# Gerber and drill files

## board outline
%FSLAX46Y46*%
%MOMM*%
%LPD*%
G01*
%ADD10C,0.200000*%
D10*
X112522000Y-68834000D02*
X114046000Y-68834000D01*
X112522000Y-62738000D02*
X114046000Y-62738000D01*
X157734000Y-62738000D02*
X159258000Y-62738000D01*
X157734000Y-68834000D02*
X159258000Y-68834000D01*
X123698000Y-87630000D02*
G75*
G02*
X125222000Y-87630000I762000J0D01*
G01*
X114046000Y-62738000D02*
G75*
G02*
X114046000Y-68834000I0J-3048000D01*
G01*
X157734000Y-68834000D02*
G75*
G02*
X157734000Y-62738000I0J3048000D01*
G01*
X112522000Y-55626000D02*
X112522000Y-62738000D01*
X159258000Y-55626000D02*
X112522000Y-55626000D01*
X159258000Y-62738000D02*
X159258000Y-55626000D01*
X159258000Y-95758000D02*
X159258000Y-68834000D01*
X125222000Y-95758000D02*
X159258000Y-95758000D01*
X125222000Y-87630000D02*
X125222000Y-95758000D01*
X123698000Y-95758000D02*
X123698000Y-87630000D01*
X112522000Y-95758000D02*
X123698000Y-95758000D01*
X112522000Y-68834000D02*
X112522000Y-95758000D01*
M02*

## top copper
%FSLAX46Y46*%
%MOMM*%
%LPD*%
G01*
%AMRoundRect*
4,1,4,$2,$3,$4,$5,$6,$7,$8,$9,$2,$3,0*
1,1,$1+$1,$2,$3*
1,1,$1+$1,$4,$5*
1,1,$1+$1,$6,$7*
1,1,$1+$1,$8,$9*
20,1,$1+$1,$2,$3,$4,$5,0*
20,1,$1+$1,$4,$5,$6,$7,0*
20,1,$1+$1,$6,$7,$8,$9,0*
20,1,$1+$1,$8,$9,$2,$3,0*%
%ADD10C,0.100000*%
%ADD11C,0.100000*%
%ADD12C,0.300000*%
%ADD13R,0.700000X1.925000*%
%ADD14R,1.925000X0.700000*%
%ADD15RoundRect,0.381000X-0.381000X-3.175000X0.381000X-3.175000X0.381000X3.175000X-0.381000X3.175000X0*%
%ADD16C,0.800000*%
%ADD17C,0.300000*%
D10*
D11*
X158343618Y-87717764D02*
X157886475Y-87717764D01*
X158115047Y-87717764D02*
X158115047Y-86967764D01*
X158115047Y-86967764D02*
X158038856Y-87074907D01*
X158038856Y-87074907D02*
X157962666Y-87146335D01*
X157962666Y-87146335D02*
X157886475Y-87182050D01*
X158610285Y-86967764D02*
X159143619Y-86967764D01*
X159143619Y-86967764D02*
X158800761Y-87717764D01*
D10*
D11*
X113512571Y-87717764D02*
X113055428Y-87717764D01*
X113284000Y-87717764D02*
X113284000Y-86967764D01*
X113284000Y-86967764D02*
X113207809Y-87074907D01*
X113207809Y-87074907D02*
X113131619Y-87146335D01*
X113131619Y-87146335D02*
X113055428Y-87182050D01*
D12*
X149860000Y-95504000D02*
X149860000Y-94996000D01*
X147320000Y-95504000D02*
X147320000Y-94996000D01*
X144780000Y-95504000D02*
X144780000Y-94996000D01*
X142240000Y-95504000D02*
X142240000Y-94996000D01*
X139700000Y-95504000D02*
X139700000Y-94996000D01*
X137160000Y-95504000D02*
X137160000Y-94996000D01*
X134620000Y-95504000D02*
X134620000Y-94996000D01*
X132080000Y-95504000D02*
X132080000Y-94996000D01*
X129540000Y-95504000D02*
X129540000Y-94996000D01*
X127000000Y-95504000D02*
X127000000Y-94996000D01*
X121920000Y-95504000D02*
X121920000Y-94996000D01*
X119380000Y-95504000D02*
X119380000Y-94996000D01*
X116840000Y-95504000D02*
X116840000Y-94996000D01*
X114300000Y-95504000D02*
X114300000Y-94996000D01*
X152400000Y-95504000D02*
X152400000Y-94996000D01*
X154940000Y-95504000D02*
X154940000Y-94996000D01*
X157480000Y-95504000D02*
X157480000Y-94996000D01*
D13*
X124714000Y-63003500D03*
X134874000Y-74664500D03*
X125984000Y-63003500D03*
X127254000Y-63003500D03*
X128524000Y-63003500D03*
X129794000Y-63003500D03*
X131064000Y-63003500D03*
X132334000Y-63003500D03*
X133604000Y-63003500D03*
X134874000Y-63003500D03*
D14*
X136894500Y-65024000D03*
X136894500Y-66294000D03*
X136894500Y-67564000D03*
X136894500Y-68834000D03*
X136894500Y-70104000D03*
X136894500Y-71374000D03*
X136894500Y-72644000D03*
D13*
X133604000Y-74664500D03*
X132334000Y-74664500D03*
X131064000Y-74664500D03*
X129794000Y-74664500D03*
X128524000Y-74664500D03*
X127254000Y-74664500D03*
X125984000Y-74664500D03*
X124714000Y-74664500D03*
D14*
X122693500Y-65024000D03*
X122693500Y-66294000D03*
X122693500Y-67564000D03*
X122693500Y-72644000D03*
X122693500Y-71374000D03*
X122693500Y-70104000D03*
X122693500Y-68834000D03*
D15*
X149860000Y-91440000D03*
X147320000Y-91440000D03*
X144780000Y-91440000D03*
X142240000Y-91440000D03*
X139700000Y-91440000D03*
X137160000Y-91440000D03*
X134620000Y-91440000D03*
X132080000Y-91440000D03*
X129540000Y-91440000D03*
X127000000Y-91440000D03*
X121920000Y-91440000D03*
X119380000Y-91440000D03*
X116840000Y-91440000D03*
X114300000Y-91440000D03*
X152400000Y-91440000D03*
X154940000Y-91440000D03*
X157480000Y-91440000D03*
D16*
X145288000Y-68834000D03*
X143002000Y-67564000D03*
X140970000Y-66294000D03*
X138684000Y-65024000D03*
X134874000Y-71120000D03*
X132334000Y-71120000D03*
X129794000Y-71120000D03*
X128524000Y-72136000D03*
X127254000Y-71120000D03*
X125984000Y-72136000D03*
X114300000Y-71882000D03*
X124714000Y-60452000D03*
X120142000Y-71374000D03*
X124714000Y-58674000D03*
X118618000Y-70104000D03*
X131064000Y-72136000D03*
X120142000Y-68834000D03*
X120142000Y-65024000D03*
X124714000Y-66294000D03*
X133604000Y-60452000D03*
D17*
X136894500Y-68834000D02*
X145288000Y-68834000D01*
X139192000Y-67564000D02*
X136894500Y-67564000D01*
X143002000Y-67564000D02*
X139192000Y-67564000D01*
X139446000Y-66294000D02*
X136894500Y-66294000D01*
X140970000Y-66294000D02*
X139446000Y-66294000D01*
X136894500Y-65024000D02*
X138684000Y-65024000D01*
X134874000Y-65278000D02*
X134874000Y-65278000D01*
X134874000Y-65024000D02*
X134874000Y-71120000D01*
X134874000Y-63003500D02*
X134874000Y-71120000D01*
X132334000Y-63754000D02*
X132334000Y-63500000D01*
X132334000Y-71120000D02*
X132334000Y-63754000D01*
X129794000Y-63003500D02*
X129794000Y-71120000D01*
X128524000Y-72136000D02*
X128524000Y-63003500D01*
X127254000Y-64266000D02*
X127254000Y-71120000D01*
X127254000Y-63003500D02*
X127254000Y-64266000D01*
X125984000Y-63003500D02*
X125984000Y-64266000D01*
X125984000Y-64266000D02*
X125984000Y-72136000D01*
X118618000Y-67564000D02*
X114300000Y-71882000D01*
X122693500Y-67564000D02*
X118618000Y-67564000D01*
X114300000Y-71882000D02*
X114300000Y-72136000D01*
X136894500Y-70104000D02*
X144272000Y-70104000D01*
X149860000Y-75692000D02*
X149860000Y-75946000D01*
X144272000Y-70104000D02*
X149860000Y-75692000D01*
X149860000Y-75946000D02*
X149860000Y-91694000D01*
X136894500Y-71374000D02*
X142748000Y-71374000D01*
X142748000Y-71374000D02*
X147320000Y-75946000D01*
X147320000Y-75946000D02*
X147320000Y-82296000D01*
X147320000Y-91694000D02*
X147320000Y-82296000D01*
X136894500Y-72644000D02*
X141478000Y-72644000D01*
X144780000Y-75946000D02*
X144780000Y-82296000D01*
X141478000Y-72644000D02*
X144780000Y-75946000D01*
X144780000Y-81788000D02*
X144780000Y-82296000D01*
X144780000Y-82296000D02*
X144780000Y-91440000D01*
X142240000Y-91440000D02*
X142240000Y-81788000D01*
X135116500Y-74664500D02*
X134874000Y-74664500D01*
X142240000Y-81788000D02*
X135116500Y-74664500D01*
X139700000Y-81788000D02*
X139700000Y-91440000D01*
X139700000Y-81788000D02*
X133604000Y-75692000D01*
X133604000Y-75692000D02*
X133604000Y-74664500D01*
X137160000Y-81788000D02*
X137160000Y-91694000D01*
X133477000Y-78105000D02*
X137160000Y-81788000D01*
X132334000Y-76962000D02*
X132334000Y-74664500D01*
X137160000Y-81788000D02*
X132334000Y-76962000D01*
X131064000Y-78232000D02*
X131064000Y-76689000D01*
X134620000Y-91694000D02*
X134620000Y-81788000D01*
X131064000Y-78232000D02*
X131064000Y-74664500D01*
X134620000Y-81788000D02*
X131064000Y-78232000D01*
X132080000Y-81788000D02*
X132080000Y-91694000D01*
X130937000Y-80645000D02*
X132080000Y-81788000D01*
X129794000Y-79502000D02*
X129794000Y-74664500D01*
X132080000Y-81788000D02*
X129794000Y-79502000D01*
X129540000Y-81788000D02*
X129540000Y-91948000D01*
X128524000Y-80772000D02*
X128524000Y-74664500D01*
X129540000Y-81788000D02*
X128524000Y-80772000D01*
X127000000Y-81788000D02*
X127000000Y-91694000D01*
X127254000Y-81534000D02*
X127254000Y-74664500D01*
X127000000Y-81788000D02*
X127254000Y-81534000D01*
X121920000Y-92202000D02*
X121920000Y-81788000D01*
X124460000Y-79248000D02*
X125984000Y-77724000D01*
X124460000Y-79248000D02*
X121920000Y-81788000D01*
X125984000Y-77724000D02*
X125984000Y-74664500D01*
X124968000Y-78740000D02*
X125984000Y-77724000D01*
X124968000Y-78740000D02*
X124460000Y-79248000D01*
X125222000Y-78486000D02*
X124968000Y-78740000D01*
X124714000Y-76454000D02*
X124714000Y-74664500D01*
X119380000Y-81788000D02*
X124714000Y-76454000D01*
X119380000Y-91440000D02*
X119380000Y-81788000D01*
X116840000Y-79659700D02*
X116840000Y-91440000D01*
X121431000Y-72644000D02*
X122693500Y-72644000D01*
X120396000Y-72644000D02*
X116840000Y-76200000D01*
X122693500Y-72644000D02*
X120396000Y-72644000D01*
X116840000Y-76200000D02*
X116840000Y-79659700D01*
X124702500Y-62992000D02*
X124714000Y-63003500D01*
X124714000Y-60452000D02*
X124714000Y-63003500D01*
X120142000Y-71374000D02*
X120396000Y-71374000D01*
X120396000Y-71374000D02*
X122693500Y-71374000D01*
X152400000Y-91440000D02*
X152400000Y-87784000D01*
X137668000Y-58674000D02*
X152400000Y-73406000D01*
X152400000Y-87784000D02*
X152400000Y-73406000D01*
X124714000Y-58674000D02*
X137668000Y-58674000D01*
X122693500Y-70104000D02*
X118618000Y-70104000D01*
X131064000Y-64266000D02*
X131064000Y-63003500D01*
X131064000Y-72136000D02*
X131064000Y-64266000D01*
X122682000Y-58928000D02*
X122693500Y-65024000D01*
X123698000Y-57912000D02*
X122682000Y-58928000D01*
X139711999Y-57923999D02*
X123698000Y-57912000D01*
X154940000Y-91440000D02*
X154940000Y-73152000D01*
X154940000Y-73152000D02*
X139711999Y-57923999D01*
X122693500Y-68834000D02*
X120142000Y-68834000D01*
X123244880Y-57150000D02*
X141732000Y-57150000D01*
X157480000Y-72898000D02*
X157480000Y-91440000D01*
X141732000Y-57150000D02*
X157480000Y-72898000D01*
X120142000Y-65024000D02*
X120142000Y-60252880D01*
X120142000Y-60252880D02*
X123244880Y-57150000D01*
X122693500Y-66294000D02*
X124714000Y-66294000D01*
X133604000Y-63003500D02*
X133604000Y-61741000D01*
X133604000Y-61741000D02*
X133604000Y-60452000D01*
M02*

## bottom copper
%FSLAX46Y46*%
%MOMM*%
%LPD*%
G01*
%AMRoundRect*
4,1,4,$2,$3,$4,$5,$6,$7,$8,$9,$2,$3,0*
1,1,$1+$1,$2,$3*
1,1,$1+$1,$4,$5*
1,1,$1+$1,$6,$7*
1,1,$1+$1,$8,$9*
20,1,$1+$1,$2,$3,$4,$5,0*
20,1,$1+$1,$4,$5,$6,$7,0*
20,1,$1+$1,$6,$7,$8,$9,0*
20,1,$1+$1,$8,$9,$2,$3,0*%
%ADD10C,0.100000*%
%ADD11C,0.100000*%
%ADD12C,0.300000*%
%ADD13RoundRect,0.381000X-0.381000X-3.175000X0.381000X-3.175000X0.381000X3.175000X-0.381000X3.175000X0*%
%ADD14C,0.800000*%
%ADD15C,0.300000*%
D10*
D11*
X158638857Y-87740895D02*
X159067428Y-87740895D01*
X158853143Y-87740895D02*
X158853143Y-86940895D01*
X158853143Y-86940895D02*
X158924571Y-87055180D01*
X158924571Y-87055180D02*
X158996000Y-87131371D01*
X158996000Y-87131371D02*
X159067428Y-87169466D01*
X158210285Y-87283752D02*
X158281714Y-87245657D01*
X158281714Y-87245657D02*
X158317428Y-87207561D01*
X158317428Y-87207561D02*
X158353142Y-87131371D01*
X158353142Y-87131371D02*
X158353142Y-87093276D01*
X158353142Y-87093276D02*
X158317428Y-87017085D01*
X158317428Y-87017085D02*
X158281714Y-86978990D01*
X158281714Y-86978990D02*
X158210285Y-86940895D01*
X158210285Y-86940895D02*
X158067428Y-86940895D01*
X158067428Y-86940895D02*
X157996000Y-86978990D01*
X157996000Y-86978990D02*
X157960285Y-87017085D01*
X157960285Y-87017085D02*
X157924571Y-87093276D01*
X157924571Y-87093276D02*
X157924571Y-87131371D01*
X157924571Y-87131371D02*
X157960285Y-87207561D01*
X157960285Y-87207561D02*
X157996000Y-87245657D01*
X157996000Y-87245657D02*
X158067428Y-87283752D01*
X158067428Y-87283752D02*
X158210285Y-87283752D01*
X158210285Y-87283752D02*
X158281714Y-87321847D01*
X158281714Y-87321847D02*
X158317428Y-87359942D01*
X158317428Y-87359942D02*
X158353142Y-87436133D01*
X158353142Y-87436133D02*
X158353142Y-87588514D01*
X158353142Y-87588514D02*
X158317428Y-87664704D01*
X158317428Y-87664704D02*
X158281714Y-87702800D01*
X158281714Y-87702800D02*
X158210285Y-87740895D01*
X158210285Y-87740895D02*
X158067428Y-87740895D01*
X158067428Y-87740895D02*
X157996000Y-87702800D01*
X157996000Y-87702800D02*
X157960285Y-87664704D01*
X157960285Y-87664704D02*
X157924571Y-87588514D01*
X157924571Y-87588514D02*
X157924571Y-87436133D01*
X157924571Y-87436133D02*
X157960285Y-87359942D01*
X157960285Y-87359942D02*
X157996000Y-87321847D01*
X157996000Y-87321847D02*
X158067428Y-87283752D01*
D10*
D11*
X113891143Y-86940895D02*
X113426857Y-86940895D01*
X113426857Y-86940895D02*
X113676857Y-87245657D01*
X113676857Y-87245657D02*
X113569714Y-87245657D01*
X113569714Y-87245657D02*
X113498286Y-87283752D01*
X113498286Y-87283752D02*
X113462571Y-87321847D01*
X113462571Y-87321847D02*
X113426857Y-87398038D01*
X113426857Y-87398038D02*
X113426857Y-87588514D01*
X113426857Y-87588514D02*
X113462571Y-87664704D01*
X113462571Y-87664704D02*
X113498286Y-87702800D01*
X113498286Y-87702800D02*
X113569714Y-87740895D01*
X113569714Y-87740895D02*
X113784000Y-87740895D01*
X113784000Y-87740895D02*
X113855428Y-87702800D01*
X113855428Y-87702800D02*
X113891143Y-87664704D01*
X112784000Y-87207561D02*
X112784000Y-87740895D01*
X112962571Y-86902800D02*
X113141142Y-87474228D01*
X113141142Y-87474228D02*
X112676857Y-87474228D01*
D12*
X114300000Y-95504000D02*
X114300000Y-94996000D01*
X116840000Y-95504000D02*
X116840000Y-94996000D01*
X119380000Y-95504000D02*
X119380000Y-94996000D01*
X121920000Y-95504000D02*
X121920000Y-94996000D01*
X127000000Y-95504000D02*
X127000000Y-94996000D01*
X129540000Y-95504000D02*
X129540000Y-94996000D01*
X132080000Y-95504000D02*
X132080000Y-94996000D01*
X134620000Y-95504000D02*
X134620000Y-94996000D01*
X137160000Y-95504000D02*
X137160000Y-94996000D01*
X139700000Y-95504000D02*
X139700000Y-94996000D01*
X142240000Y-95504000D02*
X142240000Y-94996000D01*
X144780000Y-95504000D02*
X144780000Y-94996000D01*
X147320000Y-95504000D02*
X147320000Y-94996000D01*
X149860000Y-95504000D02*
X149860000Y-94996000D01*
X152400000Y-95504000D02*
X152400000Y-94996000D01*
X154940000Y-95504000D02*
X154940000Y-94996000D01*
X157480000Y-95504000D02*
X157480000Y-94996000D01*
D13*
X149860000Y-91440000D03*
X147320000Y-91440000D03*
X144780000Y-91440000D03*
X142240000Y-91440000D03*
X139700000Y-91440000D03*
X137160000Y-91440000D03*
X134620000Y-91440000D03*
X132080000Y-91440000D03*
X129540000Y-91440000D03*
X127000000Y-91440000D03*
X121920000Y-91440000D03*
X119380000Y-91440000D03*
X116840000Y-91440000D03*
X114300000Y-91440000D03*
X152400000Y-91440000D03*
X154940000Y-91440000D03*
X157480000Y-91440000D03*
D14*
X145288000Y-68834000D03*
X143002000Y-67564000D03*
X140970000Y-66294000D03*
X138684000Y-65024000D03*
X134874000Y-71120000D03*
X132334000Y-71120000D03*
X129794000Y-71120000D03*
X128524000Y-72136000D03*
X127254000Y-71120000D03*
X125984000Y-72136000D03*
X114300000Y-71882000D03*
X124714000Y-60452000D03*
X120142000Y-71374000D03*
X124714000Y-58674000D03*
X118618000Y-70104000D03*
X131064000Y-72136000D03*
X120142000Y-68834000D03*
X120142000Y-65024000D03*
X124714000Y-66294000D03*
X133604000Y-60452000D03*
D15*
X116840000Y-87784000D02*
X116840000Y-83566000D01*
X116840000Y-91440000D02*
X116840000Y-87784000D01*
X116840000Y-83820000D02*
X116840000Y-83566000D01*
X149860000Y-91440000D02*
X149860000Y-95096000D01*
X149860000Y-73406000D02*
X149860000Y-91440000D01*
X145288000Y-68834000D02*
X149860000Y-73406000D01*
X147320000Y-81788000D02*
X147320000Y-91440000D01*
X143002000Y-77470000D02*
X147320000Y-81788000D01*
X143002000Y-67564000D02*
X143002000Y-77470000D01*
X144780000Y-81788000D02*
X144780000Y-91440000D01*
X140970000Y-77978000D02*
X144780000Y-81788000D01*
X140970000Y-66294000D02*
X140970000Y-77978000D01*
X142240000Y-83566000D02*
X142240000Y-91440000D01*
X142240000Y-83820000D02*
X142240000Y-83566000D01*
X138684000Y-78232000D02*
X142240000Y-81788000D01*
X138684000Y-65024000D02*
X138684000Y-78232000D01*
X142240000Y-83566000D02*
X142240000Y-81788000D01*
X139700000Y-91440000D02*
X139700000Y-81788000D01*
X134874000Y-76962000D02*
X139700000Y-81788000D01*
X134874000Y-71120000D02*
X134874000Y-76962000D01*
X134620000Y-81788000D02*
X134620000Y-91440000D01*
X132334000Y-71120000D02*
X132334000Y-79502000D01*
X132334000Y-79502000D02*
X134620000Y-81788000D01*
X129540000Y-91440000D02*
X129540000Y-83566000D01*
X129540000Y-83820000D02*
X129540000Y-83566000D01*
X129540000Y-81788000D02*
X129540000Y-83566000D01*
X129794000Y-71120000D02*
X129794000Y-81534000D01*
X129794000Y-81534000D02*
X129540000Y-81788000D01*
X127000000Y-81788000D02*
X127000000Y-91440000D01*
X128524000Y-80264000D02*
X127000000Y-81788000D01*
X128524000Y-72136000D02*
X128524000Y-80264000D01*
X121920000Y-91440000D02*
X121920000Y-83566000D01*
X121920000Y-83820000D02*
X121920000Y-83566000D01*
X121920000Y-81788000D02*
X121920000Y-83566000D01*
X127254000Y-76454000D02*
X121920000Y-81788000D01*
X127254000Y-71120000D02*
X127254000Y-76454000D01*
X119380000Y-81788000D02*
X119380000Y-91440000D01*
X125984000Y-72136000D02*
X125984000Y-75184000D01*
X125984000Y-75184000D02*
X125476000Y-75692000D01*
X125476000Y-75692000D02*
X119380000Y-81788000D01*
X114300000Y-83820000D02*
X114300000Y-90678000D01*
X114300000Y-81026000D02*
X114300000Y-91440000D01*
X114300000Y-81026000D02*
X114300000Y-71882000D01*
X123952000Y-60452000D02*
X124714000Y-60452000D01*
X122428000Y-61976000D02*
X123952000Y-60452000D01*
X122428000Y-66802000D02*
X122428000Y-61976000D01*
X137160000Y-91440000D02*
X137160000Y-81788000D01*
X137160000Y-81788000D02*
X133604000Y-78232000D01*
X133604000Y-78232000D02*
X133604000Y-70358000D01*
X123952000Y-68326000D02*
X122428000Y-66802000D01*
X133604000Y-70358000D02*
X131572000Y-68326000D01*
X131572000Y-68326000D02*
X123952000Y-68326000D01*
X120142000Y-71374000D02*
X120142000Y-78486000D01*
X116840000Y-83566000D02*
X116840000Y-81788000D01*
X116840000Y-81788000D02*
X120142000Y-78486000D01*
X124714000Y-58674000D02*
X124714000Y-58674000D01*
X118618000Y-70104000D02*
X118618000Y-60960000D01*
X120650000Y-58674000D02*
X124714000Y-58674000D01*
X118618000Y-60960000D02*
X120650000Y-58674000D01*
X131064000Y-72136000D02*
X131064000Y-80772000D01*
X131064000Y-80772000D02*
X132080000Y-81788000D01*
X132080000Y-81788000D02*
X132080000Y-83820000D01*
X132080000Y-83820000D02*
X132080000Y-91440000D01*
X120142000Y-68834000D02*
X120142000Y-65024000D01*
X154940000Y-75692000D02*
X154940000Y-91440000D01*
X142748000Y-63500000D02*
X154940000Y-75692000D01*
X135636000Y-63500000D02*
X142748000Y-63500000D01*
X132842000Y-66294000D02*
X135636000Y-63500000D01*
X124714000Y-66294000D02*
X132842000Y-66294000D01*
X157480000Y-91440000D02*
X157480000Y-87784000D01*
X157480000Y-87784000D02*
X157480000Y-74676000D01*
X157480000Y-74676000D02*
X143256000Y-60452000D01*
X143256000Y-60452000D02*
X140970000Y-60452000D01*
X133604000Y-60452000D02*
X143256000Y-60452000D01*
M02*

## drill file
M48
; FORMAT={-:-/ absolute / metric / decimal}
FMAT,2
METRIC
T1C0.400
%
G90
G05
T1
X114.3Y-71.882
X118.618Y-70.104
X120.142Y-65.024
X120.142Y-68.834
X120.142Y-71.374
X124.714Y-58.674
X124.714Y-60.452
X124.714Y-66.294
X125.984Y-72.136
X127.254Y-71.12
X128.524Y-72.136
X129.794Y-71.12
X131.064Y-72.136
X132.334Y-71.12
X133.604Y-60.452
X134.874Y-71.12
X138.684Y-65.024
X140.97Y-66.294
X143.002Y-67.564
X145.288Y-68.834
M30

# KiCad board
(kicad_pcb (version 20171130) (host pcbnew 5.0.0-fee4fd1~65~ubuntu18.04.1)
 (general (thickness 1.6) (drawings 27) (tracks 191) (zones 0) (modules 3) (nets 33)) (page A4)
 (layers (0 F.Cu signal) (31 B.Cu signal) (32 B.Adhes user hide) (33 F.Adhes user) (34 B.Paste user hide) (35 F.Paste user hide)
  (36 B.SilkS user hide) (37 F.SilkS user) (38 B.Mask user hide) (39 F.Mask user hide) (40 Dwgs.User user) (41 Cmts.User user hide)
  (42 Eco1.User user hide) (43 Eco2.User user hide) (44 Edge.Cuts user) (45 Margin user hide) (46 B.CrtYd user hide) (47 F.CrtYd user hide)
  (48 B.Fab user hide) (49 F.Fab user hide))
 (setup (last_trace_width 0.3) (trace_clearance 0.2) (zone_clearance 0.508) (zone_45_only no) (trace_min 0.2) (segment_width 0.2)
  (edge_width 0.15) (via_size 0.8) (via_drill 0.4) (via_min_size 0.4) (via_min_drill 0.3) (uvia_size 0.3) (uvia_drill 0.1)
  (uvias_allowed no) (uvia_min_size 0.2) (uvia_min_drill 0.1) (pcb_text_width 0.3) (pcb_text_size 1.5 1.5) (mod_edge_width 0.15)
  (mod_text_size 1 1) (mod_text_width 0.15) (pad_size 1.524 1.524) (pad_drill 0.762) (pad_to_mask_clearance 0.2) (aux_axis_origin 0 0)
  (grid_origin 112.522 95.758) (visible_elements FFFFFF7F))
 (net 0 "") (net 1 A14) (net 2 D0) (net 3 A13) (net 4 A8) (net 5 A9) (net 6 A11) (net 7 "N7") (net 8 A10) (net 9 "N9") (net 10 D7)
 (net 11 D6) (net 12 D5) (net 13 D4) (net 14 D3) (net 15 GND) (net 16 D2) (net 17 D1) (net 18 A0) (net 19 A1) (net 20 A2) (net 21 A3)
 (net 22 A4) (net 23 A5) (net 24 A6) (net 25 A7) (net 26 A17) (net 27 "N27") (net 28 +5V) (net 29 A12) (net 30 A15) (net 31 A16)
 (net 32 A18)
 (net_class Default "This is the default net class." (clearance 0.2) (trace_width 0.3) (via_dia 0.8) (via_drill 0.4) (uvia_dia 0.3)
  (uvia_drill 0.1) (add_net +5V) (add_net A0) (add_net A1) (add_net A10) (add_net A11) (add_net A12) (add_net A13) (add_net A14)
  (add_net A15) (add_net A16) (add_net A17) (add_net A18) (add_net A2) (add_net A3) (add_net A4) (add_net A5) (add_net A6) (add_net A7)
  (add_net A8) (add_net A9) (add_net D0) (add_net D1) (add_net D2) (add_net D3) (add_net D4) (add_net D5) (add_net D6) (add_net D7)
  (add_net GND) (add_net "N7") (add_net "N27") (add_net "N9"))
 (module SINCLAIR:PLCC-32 (layer F.Cu) (at 129.794 68.834 90)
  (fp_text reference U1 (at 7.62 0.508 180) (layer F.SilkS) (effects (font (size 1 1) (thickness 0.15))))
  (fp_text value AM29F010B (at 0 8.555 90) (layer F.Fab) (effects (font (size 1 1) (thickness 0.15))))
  (pad 29 smd rect (at 5.8305 -5.08 90) (size 1.925 0.7) (layers F.Cu F.Paste F.Mask) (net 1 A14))
  (pad 13 smd rect (at -5.8305 5.08 90) (size 1.925 0.7) (layers F.Cu F.Paste F.Mask) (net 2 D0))
  (pad 28 smd rect (at 5.8305 -3.81 90) (size 1.925 0.7) (layers F.Cu F.Paste F.Mask) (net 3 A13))
  (pad 27 smd rect (at 5.8305 -2.54 90) (size 1.925 0.7) (layers F.Cu F.Paste F.Mask) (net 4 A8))
  (pad 26 smd rect (at 5.8305 -1.27 90) (size 1.925 0.7) (layers F.Cu F.Paste F.Mask) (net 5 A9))
  (pad 25 smd rect (at 5.8305 0 90) (size 1.925 0.7) (layers F.Cu F.Paste F.Mask) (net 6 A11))
  (pad 24 smd rect (at 5.8305 1.27 90) (size 1.925 0.7) (layers F.Cu F.Paste F.Mask) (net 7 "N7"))
  (pad 23 smd rect (at 5.8305 2.54 90) (size 1.925 0.7) (layers F.Cu F.Paste F.Mask) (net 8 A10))
  (pad 22 smd rect (at 5.8305 3.81 90) (size 1.925 0.7) (layers F.Cu F.Paste F.Mask) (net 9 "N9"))
  (pad 21 smd rect (at 5.8305 5.08 90) (size 1.925 0.7) (layers F.Cu F.Paste F.Mask) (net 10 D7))
  (pad 20 smd rect (at 3.81 7.1005 90) (size 0.7 1.925) (layers F.Cu F.Paste F.Mask) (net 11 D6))
  (pad 19 smd rect (at 2.54 7.1005 90) (size 0.7 1.925) (layers F.Cu F.Paste F.Mask) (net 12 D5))
  (pad 18 smd rect (at 1.27 7.1005 90) (size 0.7 1.925) (layers F.Cu F.Paste F.Mask) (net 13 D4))
  (pad 17 smd rect (at 0 7.1005 90) (size 0.7 1.925) (layers F.Cu F.Paste F.Mask) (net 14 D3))
  (pad 16 smd rect (at -1.27 7.1005 90) (size 0.7 1.925) (layers F.Cu F.Paste F.Mask) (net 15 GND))
  (pad 15 smd rect (at -2.54 7.1005 90) (size 0.7 1.925) (layers F.Cu F.Paste F.Mask) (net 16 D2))
  (pad 14 smd rect (at -3.81 7.1005 90) (size 0.7 1.925) (layers F.Cu F.Paste F.Mask) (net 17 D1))
  (pad 12 smd rect (at -5.8305 3.81 90) (size 1.925 0.7) (layers F.Cu F.Paste F.Mask) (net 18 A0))
  (pad 11 smd rect (at -5.8305 2.54 90) (size 1.925 0.7) (layers F.Cu F.Paste F.Mask) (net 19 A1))
  (pad 10 smd rect (at -5.8305 1.27 90) (size 1.925 0.7) (layers F.Cu F.Paste F.Mask) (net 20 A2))
  (pad 9 smd rect (at -5.8305 0 90) (size 1.925 0.7) (layers F.Cu F.Paste F.Mask) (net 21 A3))
  (pad 8 smd rect (at -5.8305 -1.27 90) (size 1.925 0.7) (layers F.Cu F.Paste F.Mask) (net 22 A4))
  (pad 7 smd rect (at -5.8305 -2.54 90) (size 1.925 0.7) (layers F.Cu F.Paste F.Mask) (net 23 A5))
  (pad 6 smd rect (at -5.8305 -3.81 90) (size 1.925 0.7) (layers F.Cu F.Paste F.Mask) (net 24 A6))
  (pad 5 smd rect (at -5.8305 -5.08 90) (size 1.925 0.7) (layers F.Cu F.Paste F.Mask) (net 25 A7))
  (pad 30 smd rect (at 3.81 -7.1005 90) (size 0.7 1.925) (layers F.Cu F.Paste F.Mask) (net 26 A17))
  (pad 31 smd rect (at 2.54 -7.1005 90) (size 0.7 1.925) (layers F.Cu F.Paste F.Mask) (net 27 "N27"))
  (pad 32 smd rect (at 1.27 -7.1005 90) (size 0.7 1.925) (layers F.Cu F.Paste F.Mask) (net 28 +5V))
  (pad 4 smd rect (at -3.81 -7.1005 90) (size 0.7 1.925) (layers F.Cu F.Paste F.Mask) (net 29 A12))
  (pad 3 smd rect (at -2.54 -7.1005 90) (size 0.7 1.925) (layers F.Cu F.Paste F.Mask) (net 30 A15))
  (pad 2 smd rect (at -1.27 -7.1005 90) (size 0.7 1.925) (layers F.Cu F.Paste F.Mask) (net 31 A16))
  (pad 1 smd rect (at 0 -7.1005 90) (size 0.7 1.925) (layers F.Cu F.Paste F.Mask) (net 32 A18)))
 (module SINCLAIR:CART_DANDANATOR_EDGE (layer F.Cu) (at 124.46 91.44)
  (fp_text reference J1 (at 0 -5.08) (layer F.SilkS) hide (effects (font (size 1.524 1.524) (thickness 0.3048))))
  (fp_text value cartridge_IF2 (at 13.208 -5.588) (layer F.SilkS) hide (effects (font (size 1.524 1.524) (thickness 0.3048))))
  (fp_line (start -10.16 4.064) (end -10.16 3.556) (layer B.Cu) (width 0.3))
  (fp_line (start -7.62 4.064) (end -7.62 3.556) (layer B.Cu) (width 0.3))
  (fp_line (start -5.08 4.064) (end -5.08 3.556) (layer B.Cu) (width 0.3))
  (fp_line (start -2.54 4.064) (end -2.54 3.556) (layer B.Cu) (width 0.3))
  (fp_line (start 2.54 4.064) (end 2.54 3.556) (layer B.Cu) (width 0.3))
  (fp_line (start 5.08 4.064) (end 5.08 3.556) (layer B.Cu) (width 0.3))
  (fp_line (start 7.62 4.064) (end 7.62 3.556) (layer B.Cu) (width 0.3))
  (fp_line (start 10.16 4.064) (end 10.16 3.556) (layer B.Cu) (width 0.3))
  (fp_line (start 12.7 4.064) (end 12.7 3.556) (layer B.Cu) (width 0.3))
  (fp_line (start 15.24 4.064) (end 15.24 3.556) (layer B.Cu) (width 0.3))
  (fp_line (start 17.78 4.064) (end 17.78 3.556) (layer B.Cu) (width 0.3))
  (fp_line (start 20.32 4.064) (end 20.32 3.556) (layer B.Cu) (width 0.3))
  (fp_line (start 22.86 4.064) (end 22.86 3.556) (layer B.Cu) (width 0.3))
  (fp_line (start 25.4 4.064) (end 25.4 3.556) (layer B.Cu) (width 0.3))
  (fp_line (start 25.4 4.064) (end 25.4 3.556) (layer F.Cu) (width 0.3))
  (fp_line (start 22.86 4.064) (end 22.86 3.556) (layer F.Cu) (width 0.3))
  (fp_line (start 20.32 4.064) (end 20.32 3.556) (layer F.Cu) (width 0.3))
  (fp_line (start 17.78 4.064) (end 17.78 3.556) (layer F.Cu) (width 0.3))
  (fp_line (start 15.24 4.064) (end 15.24 3.556) (layer F.Cu) (width 0.3))
  (fp_line (start 12.7 4.064) (end 12.7 3.556) (layer F.Cu) (width 0.3))
  (fp_line (start 10.16 4.064) (end 10.16 3.556) (layer F.Cu) (width 0.3))
  (fp_line (start 7.62 4.064) (end 7.62 3.556) (layer F.Cu) (width 0.3))
  (fp_line (start 5.08 4.064) (end 5.08 3.556) (layer F.Cu) (width 0.3))
  (fp_line (start 2.54 4.064) (end 2.54 3.556) (layer F.Cu) (width 0.3))
  (fp_line (start -2.54 4.064) (end -2.54 3.556) (layer F.Cu) (width 0.3))
  (fp_line (start -5.08 4.064) (end -5.08 3.556) (layer F.Cu) (width 0.3))
  (fp_line (start -7.62 4.064) (end -7.62 3.556) (layer F.Cu) (width 0.3))
  (fp_line (start -10.16 4.064) (end -10.16 3.556) (layer F.Cu) (width 0.3))
  (fp_line (start 27.94 4.064) (end 27.94 3.556) (layer F.Cu) (width 0.3))
  (fp_line (start 30.48 4.064) (end 30.48 3.556) (layer F.Cu) (width 0.3))
  (fp_line (start 33.02 4.064) (end 33.02 3.556) (layer F.Cu) (width 0.3))
  (fp_line (start 27.94 4.064) (end 27.94 3.556) (layer B.Cu) (width 0.3))
  (fp_line (start 30.48 4.064) (end 30.48 3.556) (layer B.Cu) (width 0.3))
  (fp_line (start 33.02 4.064) (end 33.02 3.556) (layer B.Cu) (width 0.3))
  (pad 28 connect roundrect (at 25.4 0) (size 1.524 7.112) (layers B.Cu) (roundrect_rratio 0.25) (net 14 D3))
  (pad 26 connect roundrect (at 22.86 0) (size 1.524 7.112) (layers B.Cu) (roundrect_rratio 0.25) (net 13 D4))
  (pad 24 connect roundrect (at 20.32 0) (size 1.524 7.112) (layers B.Cu) (roundrect_rratio 0.25) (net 12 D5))
  (pad 22 connect roundrect (at 17.78 0) (size 1.524 7.112) (layers B.Cu) (roundrect_rratio 0.25) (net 11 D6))
  (pad 20 connect roundrect (at 15.24 0) (size 1.524 7.112) (layers B.Cu) (roundrect_rratio 0.25) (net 10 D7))
  (pad 18 connect roundrect (at 12.7 0) (size 1.524 7.112) (layers B.Cu) (roundrect_rratio 0.25) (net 1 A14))
  (pad 16 connect roundrect (at 10.16 0) (size 1.524 7.112) (layers B.Cu) (roundrect_rratio 0.25) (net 8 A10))
  (pad 14 connect roundrect (at 7.62 0) (size 1.524 7.112) (layers B.Cu) (roundrect_rratio 0.25) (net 7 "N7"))
  (pad 12 connect roundrect (at 5.08 0) (size 1.524 7.112) (layers B.Cu) (roundrect_rratio 0.25) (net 6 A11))
  (pad 10 connect roundrect (at 2.54 0) (size 1.524 7.112) (layers B.Cu) (roundrect_rratio 0.25) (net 5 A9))
  (pad 8 connect roundrect (at -2.54 0) (size 1.524 7.112) (layers B.Cu) (roundrect_rratio 0.25) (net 4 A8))
  (pad 6 connect roundrect (at -5.08 0) (size 1.524 7.112) (layers B.Cu) (roundrect_rratio 0.25) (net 3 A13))
  (pad 4 connect roundrect (at -7.62 0) (size 1.524 7.112) (layers B.Cu) (roundrect_rratio 0.25) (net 30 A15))
  (pad 2 connect roundrect (at -10.16 0) (size 1.524 7.112) (layers B.Cu) (roundrect_rratio 0.25) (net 28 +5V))
  (pad 27 connect roundrect (at 25.4 0) (size 1.524 7.112) (layers F.Cu) (roundrect_rratio 0.25) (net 15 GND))
  (pad 25 connect roundrect (at 22.86 0) (size 1.524 7.112) (layers F.Cu) (roundrect_rratio 0.25) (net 16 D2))
  (pad 23 connect roundrect (at 20.32 0) (size 1.524 7.112) (layers F.Cu) (roundrect_rratio 0.25) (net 17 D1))
  (pad 21 connect roundrect (at 17.78 0) (size 1.524 7.112) (layers F.Cu) (roundrect_rratio 0.25) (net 2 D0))
  (pad 19 connect roundrect (at 15.24 0) (size 1.524 7.112) (layers F.Cu) (roundrect_rratio 0.25) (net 18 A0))
  (pad 17 connect roundrect (at 12.7 0) (size 1.524 7.112) (layers F.Cu) (roundrect_rratio 0.25) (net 19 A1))
  (pad 15 connect roundrect (at 10.16 0) (size 1.524 7.112) (layers F.Cu) (roundrect_rratio 0.25) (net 20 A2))
  (pad 13 connect roundrect (at 7.62 0) (size 1.524 7.112) (layers F.Cu) (roundrect_rratio 0.25) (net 21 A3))
  (pad 11 connect roundrect (at 5.08 0) (size 1.524 7.112) (layers F.Cu) (roundrect_rratio 0.25) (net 22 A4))
  (pad 9 connect roundrect (at 2.54 0) (size 1.524 7.112) (layers F.Cu) (roundrect_rratio 0.25) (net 23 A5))
  (pad 7 connect roundrect (at -2.54 0) (size 1.524 7.112) (layers F.Cu) (roundrect_rratio 0.25) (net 24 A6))
  (pad 5 connect roundrect (at -5.08 0) (size 1.524 7.112) (layers F.Cu) (roundrect_rratio 0.25) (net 25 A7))
  (pad 3 connect roundrect (at -7.62 0) (size 1.524 7.112) (layers F.Cu) (roundrect_rratio 0.25) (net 29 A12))
  (pad 1 connect roundrect (at -10.16 0) (size 1.524 7.112) (layers F.Cu) (roundrect_rratio 0.25))
  (pad 29 connect roundrect (at 27.94 0) (size 1.524 7.112) (layers F.Cu) (roundrect_rratio 0.25) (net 31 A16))
  (pad 31 connect roundrect (at 30.48 0) (size 1.524 7.112) (layers F.Cu) (roundrect_rratio 0.25) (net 26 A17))
  (pad 33 connect roundrect (at 33.02 0) (size 1.524 7.112) (layers F.Cu) (roundrect_rratio 0.25) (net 32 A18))
  (pad 30 connect roundrect (at 27.94 0) (size 1.524 7.112) (layers B.Cu) (roundrect_rratio 0.25))
  (pad 32 connect roundrect (at 30.48 0) (size 1.524 7.112) (layers B.Cu) (roundrect_rratio 0.25) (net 27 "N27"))
  (pad 34 connect roundrect (at 33.02 0) (size 1.524 7.112) (layers B.Cu) (roundrect_rratio 0.25) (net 9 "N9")))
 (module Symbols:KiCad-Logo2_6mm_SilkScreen (layer F.Cu) (at 148.082 73.914)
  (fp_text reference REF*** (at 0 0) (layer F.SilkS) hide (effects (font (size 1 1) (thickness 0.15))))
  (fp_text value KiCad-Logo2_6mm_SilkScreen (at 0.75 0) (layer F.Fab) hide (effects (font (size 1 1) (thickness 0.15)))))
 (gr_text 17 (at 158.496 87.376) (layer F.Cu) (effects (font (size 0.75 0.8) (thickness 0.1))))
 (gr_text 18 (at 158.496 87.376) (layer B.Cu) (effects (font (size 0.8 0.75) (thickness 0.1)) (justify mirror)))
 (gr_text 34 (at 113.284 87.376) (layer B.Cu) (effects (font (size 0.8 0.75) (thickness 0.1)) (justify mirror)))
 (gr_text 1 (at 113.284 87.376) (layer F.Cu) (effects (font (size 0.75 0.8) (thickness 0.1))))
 (gr_line (start 112.522 68.834) (end 114.046 68.834) (layer Edge.Cuts) (width 0.2))
 (gr_line (start 112.522 62.738) (end 114.046 62.738) (layer Edge.Cuts) (width 0.2))
 (gr_line (start 157.734 62.738) (end 159.258 62.738) (layer Edge.Cuts) (width 0.2))
 (gr_line (start 157.734 68.834) (end 159.258 68.834) (layer Edge.Cuts) (width 0.2))
 (gr_arc (start 124.46 87.63) (end 125.222 87.63) (angle -180) (layer Edge.Cuts) (width 0.2))
 (gr_arc (start 114.046 65.786) (end 114.046 68.834) (angle -180) (layer Edge.Cuts) (width 0.2))
 (gr_arc (start 157.734 65.786) (end 157.734 62.738) (angle -180) (layer Edge.Cuts) (width 0.2))
 (gr_line (start 112.522 55.626) (end 112.522 62.738) (layer Edge.Cuts) (width 0.2))
 (gr_line (start 159.258 55.626) (end 112.522 55.626) (layer Edge.Cuts) (width 0.2))
 (gr_line (start 159.258 62.738) (end 159.258 55.626) (layer Edge.Cuts) (width 0.2))
 (gr_line (start 159.258 95.758) (end 159.258 68.834) (layer Edge.Cuts) (width 0.2))
 (gr_line (start 125.222 95.758) (end 159.258 95.758) (layer Edge.Cuts) (width 0.2))
 (gr_line (start 125.222 87.63) (end 125.222 95.758) (layer Edge.Cuts) (width 0.2))
 (gr_line (start 123.698 95.758) (end 123.698 87.63) (layer Edge.Cuts) (width 0.2))
 (gr_line (start 112.522 95.758) (end 123.698 95.758) (layer Edge.Cuts) (width 0.2))
 (gr_line (start 112.522 68.834) (end 112.522 95.758) (layer Edge.Cuts) (width 0.2))
 (segment (start 116.84 87.784) (end 116.84 83.566) (width 0.3) (layer B.Cu) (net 30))
 (segment (start 116.84 91.44) (end 116.84 87.784) (width 0.3) (layer B.Cu) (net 30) (status 10))
 (segment (start 116.84 83.82) (end 116.84 83.566) (width 0.3) (layer B.Cu) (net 30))
 (segment (start 149.86 91.44) (end 149.86 95.096) (width 0.3) (layer B.Cu) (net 14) (status 10))
 (segment (start 136.8945 68.834) (end 145.288 68.834) (width 0.3) (layer F.Cu) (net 14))
 (via (at 145.288 68.834) (size 0.8) (drill 0.4) (layers F.Cu B.Cu) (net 14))
 (segment (start 149.86 73.406) (end 149.86 91.44) (width 0.3) (layer B.Cu) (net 14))
 (segment (start 145.288 68.834) (end 149.86 73.406) (width 0.3) (layer B.Cu) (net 14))
 (segment (start 147.32 81.788) (end 147.32 91.44) (width 0.3) (layer B.Cu) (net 13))
 (segment (start 139.192 67.564) (end 136.8945 67.564) (width 0.3) (layer F.Cu) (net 13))
 (via (at 143.002 67.564) (size 0.8) (drill 0.4) (layers F.Cu B.Cu) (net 13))
 (segment (start 143.002 67.564) (end 139.192 67.564) (width 0.3) (layer F.Cu) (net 13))
 (segment (start 143.002 77.47) (end 147.32 81.788) (width 0.3) (layer B.Cu) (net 13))
 (segment (start 143.002 67.564) (end 143.002 77.47) (width 0.3) (layer B.Cu) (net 13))
 (via (at 140.97 66.294) (size 0.8) (drill 0.4) (layers F.Cu B.Cu) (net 12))
 (segment (start 139.446 66.294) (end 136.8945 66.294) (width 0.3) (layer F.Cu) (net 12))
 (segment (start 140.97 66.294) (end 139.446 66.294) (width 0.3) (layer F.Cu) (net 12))
 (segment (start 144.78 81.788) (end 144.78 91.44) (width 0.3) (layer B.Cu) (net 12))
 (segment (start 140.97 77.978) (end 144.78 81.788) (width 0.3) (layer B.Cu) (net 12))
 (segment (start 140.97 66.294) (end 140.97 77.978) (width 0.3) (layer B.Cu) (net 12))
 (segment (start 142.24 83.566) (end 142.24 91.44) (width 0.3) (layer B.Cu) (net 11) (status 20))
 (segment (start 142.24 83.82) (end 142.24 83.566) (width 0.3) (layer B.Cu) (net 11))
 (via (at 138.684 65.024) (size 0.8) (drill 0.4) (layers F.Cu B.Cu) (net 11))
 (segment (start 136.8945 65.024) (end 138.684 65.024) (width 0.3) (layer F.Cu) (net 11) (status 10))
 (segment (start 138.684 78.232) (end 142.24 81.788) (width 0.3) (layer B.Cu) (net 11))
 (segment (start 138.684 65.024) (end 138.684 78.232) (width 0.3) (layer B.Cu) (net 11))
 (segment (start 142.24 83.566) (end 142.24 81.788) (width 0.3) (layer B.Cu) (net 11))
 (segment (start 134.874 65.278) (end 134.874 65.278) (width 0.3) (layer F.Cu) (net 10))
 (segment (start 139.7 91.44) (end 139.7 81.788) (width 0.3) (layer B.Cu) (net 10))
 (segment (start 134.874 65.024) (end 134.874 71.12) (width 0.3) (layer F.Cu) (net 10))
 (via (at 134.874 71.12) (size 0.8) (drill 0.4) (layers F.Cu B.Cu) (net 10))
 (segment (start 134.874 63.0035) (end 134.874 71.12) (width 0.3) (layer F.Cu) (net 10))
 (segment (start 134.874 76.962) (end 139.7 81.788) (width 0.3) (layer B.Cu) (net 10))
 (segment (start 134.874 71.12) (end 134.874 76.962) (width 0.3) (layer B.Cu) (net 10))
 (segment (start 134.62 81.788) (end 134.62 91.44) (width 0.3) (layer B.Cu) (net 8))
 (segment (start 132.334 71.12) (end 132.334 79.502) (width 0.3) (layer B.Cu) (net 8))
 (segment (start 132.334 63.754) (end 132.334 63.5) (width 0.3) (layer F.Cu) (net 8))
 (segment (start 132.334 79.502) (end 134.62 81.788) (width 0.3) (layer B.Cu) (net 8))
 (via (at 132.334 71.12) (size 0.8) (drill 0.4) (layers F.Cu B.Cu) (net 8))
 (segment (start 132.334 71.12) (end 132.334 63.754) (width 0.3) (layer F.Cu) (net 8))
 (segment (start 129.54 91.44) (end 129.54 83.566) (width 0.3) (layer B.Cu) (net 6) (status 10))
 (segment (start 129.54 83.82) (end 129.54 83.566) (width 0.3) (layer B.Cu) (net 6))
 (segment (start 129.54 81.788) (end 129.54 83.566) (width 0.3) (layer B.Cu) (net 6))
 (segment (start 129.794 71.12) (end 129.794 81.534) (width 0.3) (layer B.Cu) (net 6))
 (via (at 129.794 71.12) (size 0.8) (drill 0.4) (layers F.Cu B.Cu) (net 6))
 (segment (start 129.794 81.534) (end 129.54 81.788) (width 0.3) (layer B.Cu) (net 6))
 (segment (start 129.794 63.0035) (end 129.794 71.12) (width 0.3) (layer F.Cu) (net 6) (status 10))
 (segment (start 127 81.788) (end 127 91.44) (width 0.3) (layer B.Cu) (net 5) (status 20))
 (segment (start 128.524 80.264) (end 127 81.788) (width 0.3) (layer B.Cu) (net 5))
 (via (at 128.524 72.136) (size 0.8) (drill 0.4) (layers F.Cu B.Cu) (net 5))
 (segment (start 128.524 72.136) (end 128.524 80.264) (width 0.3) (layer B.Cu) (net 5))
 (segment (start 128.524 72.136) (end 128.524 63.0035) (width 0.3) (layer F.Cu) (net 5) (status 20))
 (segment (start 121.92 91.44) (end 121.92 83.566) (width 0.3) (layer B.Cu) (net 4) (status 10))
 (segment (start 121.92 83.82) (end 121.92 83.566) (width 0.3) (layer B.Cu) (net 4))
 (segment (start 121.92 81.788) (end 121.92 83.566) (width 0.3) (layer B.Cu) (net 4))
 (segment (start 127.254 76.454) (end 121.92 81.788) (width 0.3) (layer B.Cu) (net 4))
 (segment (start 127.254 71.12) (end 127.254 76.454) (width 0.3) (layer B.Cu) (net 4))
 (via (at 127.254 71.12) (size 0.8) (drill 0.4) (layers F.Cu B.Cu) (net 4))
 (segment (start 127.254 64.266) (end 127.254 71.12) (width 0.3) (layer F.Cu) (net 4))
 (segment (start 127.254 63.0035) (end 127.254 64.266) (width 0.3) (layer F.Cu) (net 4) (status 10))
 (segment (start 119.38 81.788) (end 119.38 91.44) (width 0.3) (layer B.Cu) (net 3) (status 20))
 (via (at 125.984 72.136) (size 0.8) (drill 0.4) (layers F.Cu B.Cu) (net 3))
 (segment (start 125.984 63.0035) (end 125.984 64.266) (width 0.3) (layer F.Cu) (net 3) (status 10))
 (segment (start 125.984 64.266) (end 125.984 72.136) (width 0.3) (layer F.Cu) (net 3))
 (segment (start 125.984 72.136) (end 125.984 75.184) (width 0.3) (layer B.Cu) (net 3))
 (segment (start 125.984 75.184) (end 125.476 75.692) (width 0.3) (layer B.Cu) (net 3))
 (segment (start 125.476 75.692) (end 119.38 81.788) (width 0.3) (layer B.Cu) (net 3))
 (segment (start 114.3 83.82) (end 114.3 90.678) (width 0.3) (layer B.Cu) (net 28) (status 20))
 (segment (start 118.618 67.564) (end 114.3 71.882) (width 0.3) (layer F.Cu) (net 28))
 (segment (start 122.6935 67.564) (end 118.618 67.564) (width 0.3) (layer F.Cu) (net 28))
 (segment (start 114.3 81.026) (end 114.3 91.44) (width 0.3) (layer B.Cu) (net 28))
 (segment (start 114.3 71.882) (end 114.3 72.136) (width 0.3) (layer F.Cu) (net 28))
 (via (at 114.3 71.882) (size 0.8) (drill 0.4) (layers F.Cu B.Cu) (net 28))
 (segment (start 114.3 81.026) (end 114.3 71.882) (width 0.3) (layer B.Cu) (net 28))
 (segment (start 136.8945 70.104) (end 144.272 70.104) (width 0.3) (layer F.Cu) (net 15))
 (segment (start 149.86 75.692) (end 149.86 75.946) (width 0.3) (layer F.Cu) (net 15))
 (segment (start 144.272 70.104) (end 149.86 75.692) (width 0.3) (layer F.Cu) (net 15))
 (segment (start 149.86 75.946) (end 149.86 91.694) (width 0.3) (layer F.Cu) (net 15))
 (segment (start 136.8945 71.374) (end 142.748 71.374) (width 0.3) (layer F.Cu) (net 16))
 (segment (start 142.748 71.374) (end 147.32 75.946) (width 0.3) (layer F.Cu) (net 16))
 (segment (start 147.32 75.946) (end 147.32 82.296) (width 0.3) (layer F.Cu) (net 16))
 (segment (start 147.32 91.694) (end 147.32 82.296) (width 0.3) (layer F.Cu) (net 16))
 (segment (start 136.8945 72.644) (end 141.478 72.644) (width 0.3) (layer F.Cu) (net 17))
 (segment (start 144.78 75.946) (end 144.78 82.296) (width 0.3) (layer F.Cu) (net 17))
 (segment (start 141.478 72.644) (end 144.78 75.946) (width 0.3) (layer F.Cu) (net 17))
 (segment (start 144.78 81.788) (end 144.78 82.296) (width 0.3) (layer F.Cu) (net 17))
 (segment (start 144.78 82.296) (end 144.78 91.44) (width 0.3) (layer F.Cu) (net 17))
 (segment (start 142.24 91.44) (end 142.24 81.788) (width 0.3) (layer F.Cu) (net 2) (status 10))
 (segment (start 135.1165 74.6645) (end 134.874 74.6645) (width 0.3) (layer F.Cu) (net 2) (status 30))
 (segment (start 142.24 81.788) (end 135.1165 74.6645) (width 0.3) (layer F.Cu) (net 2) (status 20))
 (segment (start 139.7 81.788) (end 139.7 91.44) (width 0.3) (layer F.Cu) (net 18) (status 20))
 (segment (start 139.7 81.788) (end 133.604 75.692) (width 0.3) (layer F.Cu) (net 18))
 (segment (start 133.604 75.692) (end 133.604 74.6645) (width 0.3) (layer F.Cu) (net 18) (status 20))
 (segment (start 137.16 81.788) (end 137.16 91.694) (width 0.3) (layer F.Cu) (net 19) (status 20))
 (segment (start 133.477 78.105) (end 137.16 81.788) (width 0.3) (layer F.Cu) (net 19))
 (segment (start 132.334 76.962) (end 132.334 74.6645) (width 0.3) (layer F.Cu) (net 19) (status 20))
 (segment (start 137.16 81.788) (end 132.334 76.962) (width 0.3) (layer F.Cu) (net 19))
 (segment (start 131.064 78.232) (end 131.064 76.689) (width 0.3) (layer F.Cu) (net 20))
 (segment (start 134.62 91.694) (end 134.62 81.788) (width 0.3) (layer F.Cu) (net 20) (status 10))
 (segment (start 131.064 78.232) (end 131.064 74.6645) (width 0.3) (layer F.Cu) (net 20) (status 20))
 (segment (start 134.62 81.788) (end 131.064 78.232) (width 0.3) (layer F.Cu) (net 20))
 (segment (start 132.08 81.788) (end 132.08 91.694) (width 0.3) (layer F.Cu) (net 21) (status 20))
 (segment (start 130.937 80.645) (end 132.08 81.788) (width 0.3) (layer F.Cu) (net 21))
 (segment (start 129.794 79.502) (end 129.794 74.6645) (width 0.3) (layer F.Cu) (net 21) (status 20))
 (segment (start 132.08 81.788) (end 129.794 79.502) (width 0.3) (layer F.Cu) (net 21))
 (segment (start 129.54 81.788) (end 129.54 91.948) (width 0.3) (layer F.Cu) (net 22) (status 20))
 (segment (start 128.524 80.772) (end 128.524 74.6645) (width 0.3) (layer F.Cu) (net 22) (status 20))
 (segment (start 129.54 81.788) (end 128.524 80.772) (width 0.3) (layer F.Cu) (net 22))
 (segment (start 127 81.788) (end 127 91.694) (width 0.3) (layer F.Cu) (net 23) (status 20))
 (segment (start 127.254 81.534) (end 127.254 74.6645) (width 0.3) (layer F.Cu) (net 23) (status 20))
 (segment (start 127 81.788) (end 127.254 81.534) (width 0.3) (layer F.Cu) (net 23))
 (segment (start 121.92 92.202) (end 121.92 81.788) (width 0.3) (layer F.Cu) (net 24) (status 10))
 (segment (start 124.46 79.248) (end 125.984 77.724) (width 0.3) (layer F.Cu) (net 24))
 (segment (start 124.46 79.248) (end 121.92 81.788) (width 0.3) (layer F.Cu) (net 24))
 (segment (start 125.984 77.724) (end 125.984 74.6645) (width 0.3) (layer F.Cu) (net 24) (status 20))
 (segment (start 124.968 78.74) (end 125.984 77.724) (width 0.3) (layer F.Cu) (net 24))
 (segment (start 124.968 78.74) (end 124.46 79.248) (width 0.3) (layer F.Cu) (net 24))
 (segment (start 125.222 78.486) (end 124.968 78.74) (width 0.3) (layer F.Cu) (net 24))
 (segment (start 124.714 76.454) (end 124.714 74.6645) (width 0.3) (layer F.Cu) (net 25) (status 20))
 (segment (start 119.38 81.788) (end 124.714 76.454) (width 0.3) (layer F.Cu) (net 25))
 (segment (start 119.38 91.44) (end 119.38 81.788) (width 0.3) (layer F.Cu) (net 25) (status 10))
 (segment (start 116.84 79.6597) (end 116.84 91.44) (width 0.3) (layer F.Cu) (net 29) (status 20))
 (segment (start 121.431 72.644) (end 122.6935 72.644) (width 0.3) (layer F.Cu) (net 29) (status 20))
 (segment (start 120.396 72.644) (end 116.84 76.2) (width 0.3) (layer F.Cu) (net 29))
 (segment (start 122.6935 72.644) (end 120.396 72.644) (width 0.3) (layer F.Cu) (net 29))
 (segment (start 116.84 76.2) (end 116.84 79.6597) (width 0.3) (layer F.Cu) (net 29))
 (segment (start 124.7025 62.992) (end 124.714 63.0035) (width 0.3) (layer F.Cu) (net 1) (status 30))
 (segment (start 124.714 60.452) (end 124.714 63.0035) (width 0.3) (layer F.Cu) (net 1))
 (via (at 124.714 60.452) (size 0.8) (drill 0.4) (layers F.Cu B.Cu) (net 1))
 (segment (start 123.952 60.452) (end 124.714 60.452) (width 0.3) (layer B.Cu) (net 1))
 (segment (start 122.428 61.976) (end 123.952 60.452) (width 0.3) (layer B.Cu) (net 1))
 (segment (start 122.428 66.802) (end 122.428 61.976) (width 0.3) (layer B.Cu) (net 1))
 (segment (start 137.16 91.44) (end 137.16 81.788) (width 0.3) (layer B.Cu) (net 1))
 (segment (start 137.16 81.788) (end 133.604 78.232) (width 0.3) (layer B.Cu) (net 1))
 (segment (start 133.604 78.232) (end 133.604 70.358) (width 0.3) (layer B.Cu) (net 1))
 (segment (start 123.952 68.326) (end 122.428 66.802) (width 0.3) (layer B.Cu) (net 1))
 (segment (start 133.604 70.358) (end 131.572 68.326) (width 0.3) (layer B.Cu) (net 1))
 (segment (start 131.572 68.326) (end 123.952 68.326) (width 0.3) (layer B.Cu) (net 1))
 (segment (start 120.142 71.374) (end 120.396 71.374) (width 0.3) (layer F.Cu) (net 30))
 (segment (start 120.396 71.374) (end 122.6935 71.374) (width 0.3) (layer F.Cu) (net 30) (status 20))
 (via (at 120.142 71.374) (size 0.8) (drill 0.4) (layers F.Cu B.Cu) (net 30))
 (segment (start 120.142 71.374) (end 120.142 78.486) (width 0.3) (layer B.Cu) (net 30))
 (segment (start 116.84 83.566) (end 116.84 81.788) (width 0.3) (layer B.Cu) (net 30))
 (segment (start 116.84 81.788) (end 120.142 78.486) (width 0.3) (layer B.Cu) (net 30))
 (segment (start 152.4 91.44) (end 152.4 87.784) (width 0.3) (layer F.Cu) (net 31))
 (segment (start 124.714 58.674) (end 124.714 58.674) (width 0.3) (layer B.Cu) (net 31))
 (via (at 124.714 58.674) (size 0.8) (drill 0.4) (layers F.Cu B.Cu) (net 31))
 (segment (start 137.668 58.674) (end 152.4 73.406) (width 0.3) (layer F.Cu) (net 31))
 (segment (start 152.4 87.784) (end 152.4 73.406) (width 0.3) (layer F.Cu) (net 31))
 (segment (start 124.714 58.674) (end 137.668 58.674) (width 0.3) (layer F.Cu) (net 31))
 (via (at 118.618 70.104) (size 0.8) (drill 0.4) (layers F.Cu B.Cu) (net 31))
 (segment (start 122.6935 70.104) (end 118.618 70.104) (width 0.3) (layer F.Cu) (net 31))
 (segment (start 118.618 70.104) (end 118.618 60.96) (width 0.3) (layer B.Cu) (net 31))
 (segment (start 120.65 58.674) (end 124.714 58.674) (width 0.3) (layer B.Cu) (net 31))
 (segment (start 118.618 60.96) (end 120.65 58.674) (width 0.3) (layer B.Cu) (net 31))
 (segment (start 131.064 64.266) (end 131.064 63.0035) (width 0.3) (layer F.Cu) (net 7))
 (segment (start 131.064 72.136) (end 131.064 80.772) (width 0.3) (layer B.Cu) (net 7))
 (via (at 131.064 72.136) (size 0.8) (drill 0.4) (layers F.Cu B.Cu) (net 7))
 (segment (start 131.064 80.772) (end 132.08 81.788) (width 0.3) (layer B.Cu) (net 7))
 (segment (start 132.08 81.788) (end 132.08 83.82) (width 0.3) (layer B.Cu) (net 7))
 (segment (start 132.08 83.82) (end 132.08 91.44) (width 0.3) (layer B.Cu) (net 7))
 (segment (start 131.064 72.136) (end 131.064 64.266) (width 0.3) (layer F.Cu) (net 7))
 (segment (start 122.682 58.928) (end 122.6935 65.024) (width 0.3) (layer F.Cu) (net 26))
 (segment (start 123.698 57.912) (end 122.682 58.928) (width 0.3) (layer F.Cu) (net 26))
 (segment (start 139.711999 57.923999) (end 123.698 57.912) (width 0.3) (layer F.Cu) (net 26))
 (segment (start 154.94 91.44) (end 154.94 73.152) (width 0.3) (layer F.Cu) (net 26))
 (segment (start 154.94 73.152) (end 139.711999 57.923999) (width 0.3) (layer F.Cu) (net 26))
 (segment (start 122.6935 68.834) (end 120.142 68.834) (width 0.3) (layer F.Cu) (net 32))
 (via (at 120.142 68.834) (size 0.8) (drill 0.4) (layers F.Cu B.Cu) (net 32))
 (segment (start 120.142 68.834) (end 120.142 65.024) (width 0.3) (layer B.Cu) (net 32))
 (segment (start 123.24488 57.15) (end 141.732 57.15) (width 0.3) (layer F.Cu) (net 32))
 (via (at 120.142 65.024) (size 0.8) (drill 0.4) (layers F.Cu B.Cu) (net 32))
 (segment (start 157.48 72.898) (end 157.48 91.44) (width 0.3) (layer F.Cu) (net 32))
 (segment (start 141.732 57.15) (end 157.48 72.898) (width 0.3) (layer F.Cu) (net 32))
 (segment (start 120.142 65.024) (end 120.142 60.25288) (width 0.3) (layer F.Cu) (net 32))
 (segment (start 120.142 60.25288) (end 123.24488 57.15) (width 0.3) (layer F.Cu) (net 32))
 (segment (start 122.6935 66.294) (end 124.714 66.294) (width 0.3) (layer F.Cu) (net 27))
 (via (at 124.714 66.294) (size 0.8) (drill 0.4) (layers F.Cu B.Cu) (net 27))
 (segment (start 154.94 75.692) (end 154.94 91.44) (width 0.3) (layer B.Cu) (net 27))
 (segment (start 142.748 63.5) (end 154.94 75.692) (width 0.3) (layer B.Cu) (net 27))
 (segment (start 135.636 63.5) (end 142.748 63.5) (width 0.3) (layer B.Cu) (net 27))
 (segment (start 132.842 66.294) (end 135.636 63.5) (width 0.3) (layer B.Cu) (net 27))
 (segment (start 124.714 66.294) (end 132.842 66.294) (width 0.3) (layer B.Cu) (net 27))
 (segment (start 157.48 91.44) (end 157.48 87.784) (width 0.3) (layer B.Cu) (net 9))
 (segment (start 157.48 87.784) (end 157.48 74.676) (width 0.3) (layer B.Cu) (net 9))
 (segment (start 157.48 74.676) (end 143.256 60.452) (width 0.3) (layer B.Cu) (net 9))
 (segment (start 143.256 60.452) (end 140.97 60.452) (width 0.3) (layer B.Cu) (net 9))
 (segment (start 133.604 63.0035) (end 133.604 61.741) (width 0.3) (layer F.Cu) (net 9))
 (segment (start 133.604 61.741) (end 133.604 60.452) (width 0.3) (layer F.Cu) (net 9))
 (via (at 133.604 60.452) (size 0.8) (drill 0.4) (layers F.Cu B.Cu) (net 9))
 (segment (start 133.604 60.452) (end 143.256 60.452) (width 0.3) (layer B.Cu) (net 9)))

